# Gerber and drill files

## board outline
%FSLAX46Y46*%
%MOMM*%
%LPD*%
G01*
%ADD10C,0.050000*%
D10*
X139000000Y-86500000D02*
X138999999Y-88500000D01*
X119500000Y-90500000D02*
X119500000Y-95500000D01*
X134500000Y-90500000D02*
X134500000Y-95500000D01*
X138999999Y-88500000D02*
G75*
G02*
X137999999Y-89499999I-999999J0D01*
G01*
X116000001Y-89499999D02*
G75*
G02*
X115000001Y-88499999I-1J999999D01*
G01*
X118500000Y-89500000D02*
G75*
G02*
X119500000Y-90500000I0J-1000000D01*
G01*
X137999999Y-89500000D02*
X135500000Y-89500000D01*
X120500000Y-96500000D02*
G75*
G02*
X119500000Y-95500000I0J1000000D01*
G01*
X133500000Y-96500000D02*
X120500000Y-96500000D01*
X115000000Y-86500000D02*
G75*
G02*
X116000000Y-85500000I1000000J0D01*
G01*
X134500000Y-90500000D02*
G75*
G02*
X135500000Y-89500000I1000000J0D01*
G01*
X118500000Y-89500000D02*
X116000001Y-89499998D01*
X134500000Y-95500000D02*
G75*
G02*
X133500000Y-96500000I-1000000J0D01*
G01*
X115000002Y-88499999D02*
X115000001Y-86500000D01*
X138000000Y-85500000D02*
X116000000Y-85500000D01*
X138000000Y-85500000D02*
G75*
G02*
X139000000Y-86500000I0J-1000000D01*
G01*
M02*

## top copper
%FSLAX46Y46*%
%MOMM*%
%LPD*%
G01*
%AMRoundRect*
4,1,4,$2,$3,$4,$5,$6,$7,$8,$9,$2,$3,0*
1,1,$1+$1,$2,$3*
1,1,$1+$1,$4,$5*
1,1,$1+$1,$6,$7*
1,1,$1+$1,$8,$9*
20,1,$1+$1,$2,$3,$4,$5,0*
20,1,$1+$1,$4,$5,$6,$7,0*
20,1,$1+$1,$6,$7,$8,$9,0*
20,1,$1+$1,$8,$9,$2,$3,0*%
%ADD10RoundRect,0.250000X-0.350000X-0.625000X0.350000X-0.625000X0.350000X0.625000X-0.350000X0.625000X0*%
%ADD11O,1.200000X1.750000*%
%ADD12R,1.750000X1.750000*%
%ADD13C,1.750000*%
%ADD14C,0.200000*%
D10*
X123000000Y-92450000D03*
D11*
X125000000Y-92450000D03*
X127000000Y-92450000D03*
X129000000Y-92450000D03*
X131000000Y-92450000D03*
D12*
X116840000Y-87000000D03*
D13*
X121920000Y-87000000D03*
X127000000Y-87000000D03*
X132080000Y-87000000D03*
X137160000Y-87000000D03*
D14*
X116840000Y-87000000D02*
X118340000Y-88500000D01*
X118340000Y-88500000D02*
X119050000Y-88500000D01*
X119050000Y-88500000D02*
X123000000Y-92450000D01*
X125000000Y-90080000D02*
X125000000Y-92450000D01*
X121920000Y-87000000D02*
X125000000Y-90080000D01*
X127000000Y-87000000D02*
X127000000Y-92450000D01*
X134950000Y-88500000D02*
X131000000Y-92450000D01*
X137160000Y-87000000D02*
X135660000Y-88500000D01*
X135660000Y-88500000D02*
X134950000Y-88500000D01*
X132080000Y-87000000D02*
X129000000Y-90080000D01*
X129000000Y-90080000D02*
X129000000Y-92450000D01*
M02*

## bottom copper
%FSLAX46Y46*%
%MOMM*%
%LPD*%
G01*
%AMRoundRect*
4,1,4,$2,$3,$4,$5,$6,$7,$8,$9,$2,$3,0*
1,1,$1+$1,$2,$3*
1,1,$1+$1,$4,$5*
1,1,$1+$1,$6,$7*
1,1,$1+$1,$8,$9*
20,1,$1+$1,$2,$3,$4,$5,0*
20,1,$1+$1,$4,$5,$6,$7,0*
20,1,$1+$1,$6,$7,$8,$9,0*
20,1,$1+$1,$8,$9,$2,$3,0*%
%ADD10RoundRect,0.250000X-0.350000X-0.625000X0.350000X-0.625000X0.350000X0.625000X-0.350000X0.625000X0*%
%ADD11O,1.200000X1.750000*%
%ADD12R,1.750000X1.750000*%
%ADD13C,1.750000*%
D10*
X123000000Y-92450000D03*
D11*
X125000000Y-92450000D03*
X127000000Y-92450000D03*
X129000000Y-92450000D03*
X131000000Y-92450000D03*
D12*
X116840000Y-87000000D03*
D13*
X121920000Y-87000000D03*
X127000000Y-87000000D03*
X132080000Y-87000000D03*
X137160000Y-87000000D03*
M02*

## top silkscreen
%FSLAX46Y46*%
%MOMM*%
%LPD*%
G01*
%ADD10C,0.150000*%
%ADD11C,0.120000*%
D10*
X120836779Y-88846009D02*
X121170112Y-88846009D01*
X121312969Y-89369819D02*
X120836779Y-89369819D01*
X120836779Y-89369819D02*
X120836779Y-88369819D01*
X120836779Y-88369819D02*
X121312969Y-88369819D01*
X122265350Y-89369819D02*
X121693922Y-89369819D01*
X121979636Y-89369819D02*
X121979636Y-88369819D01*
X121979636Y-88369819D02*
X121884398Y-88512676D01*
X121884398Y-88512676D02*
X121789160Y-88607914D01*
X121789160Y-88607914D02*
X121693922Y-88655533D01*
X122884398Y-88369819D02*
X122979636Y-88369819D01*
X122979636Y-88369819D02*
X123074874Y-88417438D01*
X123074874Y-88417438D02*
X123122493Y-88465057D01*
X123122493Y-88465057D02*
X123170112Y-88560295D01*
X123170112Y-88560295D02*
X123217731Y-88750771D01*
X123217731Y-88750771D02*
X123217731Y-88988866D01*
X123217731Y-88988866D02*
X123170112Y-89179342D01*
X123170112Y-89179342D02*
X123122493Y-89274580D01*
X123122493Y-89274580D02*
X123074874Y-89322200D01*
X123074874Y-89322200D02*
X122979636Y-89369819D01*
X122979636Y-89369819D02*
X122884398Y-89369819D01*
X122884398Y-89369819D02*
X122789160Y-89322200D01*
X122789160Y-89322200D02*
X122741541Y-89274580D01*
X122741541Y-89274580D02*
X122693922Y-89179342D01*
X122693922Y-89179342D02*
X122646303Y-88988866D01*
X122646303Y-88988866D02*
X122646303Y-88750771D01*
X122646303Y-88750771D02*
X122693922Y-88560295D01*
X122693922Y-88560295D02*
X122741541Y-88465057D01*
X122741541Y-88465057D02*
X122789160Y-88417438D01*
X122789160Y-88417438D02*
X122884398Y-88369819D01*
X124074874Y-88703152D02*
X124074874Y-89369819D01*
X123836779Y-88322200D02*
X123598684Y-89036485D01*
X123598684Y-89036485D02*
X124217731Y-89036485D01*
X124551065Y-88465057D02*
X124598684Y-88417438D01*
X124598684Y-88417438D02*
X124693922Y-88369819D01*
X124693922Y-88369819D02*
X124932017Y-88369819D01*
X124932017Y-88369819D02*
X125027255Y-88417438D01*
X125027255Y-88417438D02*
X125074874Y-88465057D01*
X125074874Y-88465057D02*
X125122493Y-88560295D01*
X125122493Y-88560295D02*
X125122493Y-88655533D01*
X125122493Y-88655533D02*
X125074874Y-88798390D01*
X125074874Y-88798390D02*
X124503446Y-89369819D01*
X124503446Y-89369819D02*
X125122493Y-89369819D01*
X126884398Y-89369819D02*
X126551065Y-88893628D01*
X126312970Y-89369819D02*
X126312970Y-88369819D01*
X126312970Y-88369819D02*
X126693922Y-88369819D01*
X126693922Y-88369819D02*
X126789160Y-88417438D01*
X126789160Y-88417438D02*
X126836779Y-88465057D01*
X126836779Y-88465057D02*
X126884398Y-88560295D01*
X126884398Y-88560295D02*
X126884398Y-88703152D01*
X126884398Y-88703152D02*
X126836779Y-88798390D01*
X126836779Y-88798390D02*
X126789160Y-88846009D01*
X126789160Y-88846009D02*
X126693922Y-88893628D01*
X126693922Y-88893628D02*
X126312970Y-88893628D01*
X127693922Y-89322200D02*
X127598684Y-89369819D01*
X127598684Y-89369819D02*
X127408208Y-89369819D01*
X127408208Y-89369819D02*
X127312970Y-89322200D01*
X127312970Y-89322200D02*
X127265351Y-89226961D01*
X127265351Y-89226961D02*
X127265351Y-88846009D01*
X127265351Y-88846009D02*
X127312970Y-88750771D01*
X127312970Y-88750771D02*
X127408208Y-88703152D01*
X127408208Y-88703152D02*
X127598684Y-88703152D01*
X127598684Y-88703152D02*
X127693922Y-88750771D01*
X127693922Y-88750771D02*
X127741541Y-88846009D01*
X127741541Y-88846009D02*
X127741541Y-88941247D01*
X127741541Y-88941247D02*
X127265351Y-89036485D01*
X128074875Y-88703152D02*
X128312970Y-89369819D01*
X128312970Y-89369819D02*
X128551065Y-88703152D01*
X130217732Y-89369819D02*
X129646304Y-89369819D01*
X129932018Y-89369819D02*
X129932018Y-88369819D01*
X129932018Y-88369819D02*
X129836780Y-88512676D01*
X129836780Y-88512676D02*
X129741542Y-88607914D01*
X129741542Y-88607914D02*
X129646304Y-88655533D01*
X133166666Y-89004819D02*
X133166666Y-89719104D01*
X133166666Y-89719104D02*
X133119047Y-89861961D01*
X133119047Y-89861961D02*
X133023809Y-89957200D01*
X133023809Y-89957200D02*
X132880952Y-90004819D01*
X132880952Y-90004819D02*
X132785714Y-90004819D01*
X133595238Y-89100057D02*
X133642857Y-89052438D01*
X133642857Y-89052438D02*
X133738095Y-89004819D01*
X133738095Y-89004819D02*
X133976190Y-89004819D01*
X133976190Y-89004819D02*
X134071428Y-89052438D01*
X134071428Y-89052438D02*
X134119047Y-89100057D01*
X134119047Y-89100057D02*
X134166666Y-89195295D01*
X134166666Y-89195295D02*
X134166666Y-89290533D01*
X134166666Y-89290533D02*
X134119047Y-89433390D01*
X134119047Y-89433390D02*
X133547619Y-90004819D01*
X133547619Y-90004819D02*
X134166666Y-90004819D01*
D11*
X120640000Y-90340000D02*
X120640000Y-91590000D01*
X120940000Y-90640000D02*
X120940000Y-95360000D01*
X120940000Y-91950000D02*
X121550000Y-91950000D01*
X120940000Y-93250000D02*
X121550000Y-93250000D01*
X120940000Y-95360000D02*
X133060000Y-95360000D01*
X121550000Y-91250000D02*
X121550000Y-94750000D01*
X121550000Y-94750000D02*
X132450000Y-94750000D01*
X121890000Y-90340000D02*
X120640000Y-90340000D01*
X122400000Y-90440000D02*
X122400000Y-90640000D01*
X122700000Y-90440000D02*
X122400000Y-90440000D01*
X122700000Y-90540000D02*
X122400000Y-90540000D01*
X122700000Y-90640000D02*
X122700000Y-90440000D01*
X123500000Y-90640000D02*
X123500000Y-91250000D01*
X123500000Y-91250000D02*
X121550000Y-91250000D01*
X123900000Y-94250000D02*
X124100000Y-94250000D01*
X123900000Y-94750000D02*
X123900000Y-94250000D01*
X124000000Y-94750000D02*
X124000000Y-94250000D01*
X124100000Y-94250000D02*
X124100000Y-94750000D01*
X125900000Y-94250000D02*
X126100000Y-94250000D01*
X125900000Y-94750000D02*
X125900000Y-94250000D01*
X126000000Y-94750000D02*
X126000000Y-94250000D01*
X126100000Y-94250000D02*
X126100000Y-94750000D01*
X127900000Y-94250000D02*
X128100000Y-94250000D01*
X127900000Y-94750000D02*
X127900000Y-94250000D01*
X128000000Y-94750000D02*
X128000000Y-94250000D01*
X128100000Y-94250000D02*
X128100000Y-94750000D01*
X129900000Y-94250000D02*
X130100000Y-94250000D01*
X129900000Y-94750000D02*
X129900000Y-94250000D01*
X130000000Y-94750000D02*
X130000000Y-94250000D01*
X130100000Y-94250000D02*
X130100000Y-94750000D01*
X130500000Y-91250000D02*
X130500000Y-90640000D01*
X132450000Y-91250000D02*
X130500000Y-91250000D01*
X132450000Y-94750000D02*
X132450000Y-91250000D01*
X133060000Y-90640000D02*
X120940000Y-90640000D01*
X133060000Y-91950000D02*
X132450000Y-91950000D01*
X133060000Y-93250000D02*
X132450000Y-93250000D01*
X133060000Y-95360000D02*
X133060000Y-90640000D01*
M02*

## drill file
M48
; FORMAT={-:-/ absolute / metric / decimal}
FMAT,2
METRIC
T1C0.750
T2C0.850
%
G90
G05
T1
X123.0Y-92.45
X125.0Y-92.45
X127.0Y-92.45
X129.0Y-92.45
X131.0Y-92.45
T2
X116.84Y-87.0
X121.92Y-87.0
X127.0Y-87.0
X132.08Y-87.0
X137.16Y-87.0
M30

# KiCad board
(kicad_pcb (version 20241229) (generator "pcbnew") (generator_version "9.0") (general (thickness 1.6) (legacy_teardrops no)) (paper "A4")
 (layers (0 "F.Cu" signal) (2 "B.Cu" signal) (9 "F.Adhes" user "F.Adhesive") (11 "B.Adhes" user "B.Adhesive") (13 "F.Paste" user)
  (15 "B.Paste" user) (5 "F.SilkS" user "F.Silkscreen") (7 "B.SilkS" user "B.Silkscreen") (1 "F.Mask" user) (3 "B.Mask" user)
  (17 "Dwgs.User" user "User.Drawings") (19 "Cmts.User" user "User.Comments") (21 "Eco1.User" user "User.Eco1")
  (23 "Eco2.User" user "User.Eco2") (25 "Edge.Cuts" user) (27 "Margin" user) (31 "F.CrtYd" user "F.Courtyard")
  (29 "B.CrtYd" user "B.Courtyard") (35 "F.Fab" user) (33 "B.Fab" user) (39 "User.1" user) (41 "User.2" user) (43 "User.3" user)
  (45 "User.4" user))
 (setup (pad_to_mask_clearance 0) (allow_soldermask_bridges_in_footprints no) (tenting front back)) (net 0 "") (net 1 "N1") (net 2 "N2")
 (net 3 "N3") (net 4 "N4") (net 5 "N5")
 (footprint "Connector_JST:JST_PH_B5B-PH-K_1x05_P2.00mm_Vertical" (layer "F.Cu") (at 123 92.45)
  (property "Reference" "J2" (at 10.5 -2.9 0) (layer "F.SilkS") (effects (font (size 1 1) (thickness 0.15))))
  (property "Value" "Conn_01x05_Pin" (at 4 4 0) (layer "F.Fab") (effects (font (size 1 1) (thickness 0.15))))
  (fp_line (start -2.36 -2.11) (end -2.36 -0.86) (stroke (width 0.12) (type solid)) (layer "F.SilkS"))
  (fp_line (start -2.06 -1.81) (end -2.06 2.91) (stroke (width 0.12) (type solid)) (layer "F.SilkS"))
  (fp_line (start -2.06 -0.5) (end -1.45 -0.5) (stroke (width 0.12) (type solid)) (layer "F.SilkS"))
  (fp_line (start -2.06 0.8) (end -1.45 0.8) (stroke (width 0.12) (type solid)) (layer "F.SilkS"))
  (fp_line (start -2.06 2.91) (end 10.06 2.91) (stroke (width 0.12) (type solid)) (layer "F.SilkS"))
  (fp_line (start -1.45 -1.2) (end -1.45 2.3) (stroke (width 0.12) (type solid)) (layer "F.SilkS"))
  (fp_line (start -1.45 2.3) (end 9.45 2.3) (stroke (width 0.12) (type solid)) (layer "F.SilkS"))
  (fp_line (start -1.11 -2.11) (end -2.36 -2.11) (stroke (width 0.12) (type solid)) (layer "F.SilkS"))
  (fp_line (start -0.6 -2.01) (end -0.6 -1.81) (stroke (width 0.12) (type solid)) (layer "F.SilkS"))
  (fp_line (start -0.3 -2.01) (end -0.6 -2.01) (stroke (width 0.12) (type solid)) (layer "F.SilkS"))
  (fp_line (start -0.3 -1.91) (end -0.6 -1.91) (stroke (width 0.12) (type solid)) (layer "F.SilkS"))
  (fp_line (start -0.3 -1.81) (end -0.3 -2.01) (stroke (width 0.12) (type solid)) (layer "F.SilkS"))
  (fp_line (start 0.5 -1.81) (end 0.5 -1.2) (stroke (width 0.12) (type solid)) (layer "F.SilkS"))
  (fp_line (start 0.5 -1.2) (end -1.45 -1.2) (stroke (width 0.12) (type solid)) (layer "F.SilkS"))
  (fp_line (start 0.9 1.8) (end 1.1 1.8) (stroke (width 0.12) (type solid)) (layer "F.SilkS"))
  (fp_line (start 0.9 2.3) (end 0.9 1.8) (stroke (width 0.12) (type solid)) (layer "F.SilkS"))
  (fp_line (start 1 2.3) (end 1 1.8) (stroke (width 0.12) (type solid)) (layer "F.SilkS"))
  (fp_line (start 1.1 1.8) (end 1.1 2.3) (stroke (width 0.12) (type solid)) (layer "F.SilkS"))
  (fp_line (start 2.9 1.8) (end 3.1 1.8) (stroke (width 0.12) (type solid)) (layer "F.SilkS"))
  (fp_line (start 2.9 2.3) (end 2.9 1.8) (stroke (width 0.12) (type solid)) (layer "F.SilkS"))
  (fp_line (start 3 2.3) (end 3 1.8) (stroke (width 0.12) (type solid)) (layer "F.SilkS"))
  (fp_line (start 3.1 1.8) (end 3.1 2.3) (stroke (width 0.12) (type solid)) (layer "F.SilkS"))
  (fp_line (start 4.9 1.8) (end 5.1 1.8) (stroke (width 0.12) (type solid)) (layer "F.SilkS"))
  (fp_line (start 4.9 2.3) (end 4.9 1.8) (stroke (width 0.12) (type solid)) (layer "F.SilkS"))
  (fp_line (start 5 2.3) (end 5 1.8) (stroke (width 0.12) (type solid)) (layer "F.SilkS"))
  (fp_line (start 5.1 1.8) (end 5.1 2.3) (stroke (width 0.12) (type solid)) (layer "F.SilkS"))
  (fp_line (start 6.9 1.8) (end 7.1 1.8) (stroke (width 0.12) (type solid)) (layer "F.SilkS"))
  (fp_line (start 6.9 2.3) (end 6.9 1.8) (stroke (width 0.12) (type solid)) (layer "F.SilkS"))
  (fp_line (start 7 2.3) (end 7 1.8) (stroke (width 0.12) (type solid)) (layer "F.SilkS"))
  (fp_line (start 7.1 1.8) (end 7.1 2.3) (stroke (width 0.12) (type solid)) (layer "F.SilkS"))
  (fp_line (start 7.5 -1.2) (end 7.5 -1.81) (stroke (width 0.12) (type solid)) (layer "F.SilkS"))
  (fp_line (start 9.45 -1.2) (end 7.5 -1.2) (stroke (width 0.12) (type solid)) (layer "F.SilkS"))
  (fp_line (start 9.45 2.3) (end 9.45 -1.2) (stroke (width 0.12) (type solid)) (layer "F.SilkS"))
  (fp_line (start 10.06 -1.81) (end -2.06 -1.81) (stroke (width 0.12) (type solid)) (layer "F.SilkS"))
  (fp_line (start 10.06 -0.5) (end 9.45 -0.5) (stroke (width 0.12) (type solid)) (layer "F.SilkS"))
  (fp_line (start 10.06 0.8) (end 9.45 0.8) (stroke (width 0.12) (type solid)) (layer "F.SilkS"))
  (fp_line (start 10.06 2.91) (end 10.06 -1.81) (stroke (width 0.12) (type solid)) (layer "F.SilkS"))
  (pad "1" thru_hole roundrect (at 0 0) (size 1.2 1.75) (drill 0.75) (layers "*.Cu" "*.Mask") (remove_unused_layers no)
   (roundrect_rratio 0.208333) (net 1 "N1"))
  (pad "2" thru_hole oval (at 2 0) (size 1.2 1.75) (drill 0.75) (layers "*.Cu" "*.Mask") (remove_unused_layers no) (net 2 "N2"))
  (pad "3" thru_hole oval (at 4 0) (size 1.2 1.75) (drill 0.75) (layers "*.Cu" "*.Mask") (remove_unused_layers no) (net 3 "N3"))
  (pad "4" thru_hole oval (at 6 0) (size 1.2 1.75) (drill 0.75) (layers "*.Cu" "*.Mask") (remove_unused_layers no) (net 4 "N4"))
  (pad "5" thru_hole oval (at 8 0) (size 1.2 1.75) (drill 0.75) (layers "*.Cu" "*.Mask") (remove_unused_layers no) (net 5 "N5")))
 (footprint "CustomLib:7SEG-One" (layer "B.Cu") (at 116.84 87)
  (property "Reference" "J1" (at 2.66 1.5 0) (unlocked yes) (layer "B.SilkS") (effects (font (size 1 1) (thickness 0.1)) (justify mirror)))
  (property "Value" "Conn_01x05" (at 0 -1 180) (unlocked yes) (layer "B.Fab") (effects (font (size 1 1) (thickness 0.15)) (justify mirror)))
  (pad "1" thru_hole rect (at 0 0) (size 1.75 1.75) (drill 0.85) (layers "*.Cu" "*.Mask") (remove_unused_layers no) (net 1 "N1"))
  (pad "2" thru_hole circle (at 5.08 0) (size 1.75 1.75) (drill 0.85) (layers "*.Cu" "*.Mask") (remove_unused_layers no) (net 2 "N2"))
  (pad "3" thru_hole circle (at 10.16 0) (size 1.75 1.75) (drill 0.85) (layers "*.Cu" "*.Mask") (remove_unused_layers no) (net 3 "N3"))
  (pad "4" thru_hole circle (at 15.24 0) (size 1.75 1.75) (drill 0.85) (layers "*.Cu" "*.Mask") (remove_unused_layers no) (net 4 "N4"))
  (pad "5" thru_hole circle (at 20.32 0) (size 1.75 1.75) (drill 0.85) (layers "*.Cu" "*.Mask") (remove_unused_layers no) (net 5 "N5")))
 (gr_line (start 139 86.5) (end 138.999999 88.5) (stroke (width 0.05) (type default)) (layer "Edge.Cuts"))
 (gr_line (start 119.5 90.5) (end 119.5 95.5) (stroke (width 0.05) (type default)) (layer "Edge.Cuts"))
 (gr_line (start 134.5 90.5) (end 134.5 95.5) (stroke (width 0.05) (type default)) (layer "Edge.Cuts"))
 (gr_arc (start 138.999999 88.5) (mid 138.707106 89.207107) (end 137.999999 89.5) (stroke (width 0.05) (type default)) (layer "Edge.Cuts"))
 (gr_arc (start 116.000001 89.499999) (mid 115.292894 89.207106) (end 115.000001 88.499999) (stroke (width 0.05) (type default))
  (layer "Edge.Cuts"))
 (gr_arc (start 118.5 89.5) (mid 119.207107 89.792893) (end 119.5 90.5) (stroke (width 0.05) (type default)) (layer "Edge.Cuts"))
 (gr_line (start 137.999999 89.5) (end 135.5 89.5) (stroke (width 0.05) (type default)) (layer "Edge.Cuts"))
 (gr_arc (start 120.5 96.5) (mid 119.792893 96.207107) (end 119.5 95.5) (stroke (width 0.05) (type default)) (layer "Edge.Cuts"))
 (gr_line (start 133.5 96.5) (end 120.5 96.5) (stroke (width 0.05) (type default)) (layer "Edge.Cuts"))
 (gr_arc (start 115 86.5) (mid 115.292893 85.792893) (end 116 85.5) (stroke (width 0.05) (type default)) (layer "Edge.Cuts"))
 (gr_arc (start 134.5 90.5) (mid 134.792893 89.792893) (end 135.5 89.5) (stroke (width 0.05) (type default)) (layer "Edge.Cuts"))
 (gr_line (start 118.5 89.5) (end 116.000001 89.499998) (stroke (width 0.05) (type default)) (layer "Edge.Cuts"))
 (gr_arc (start 134.5 95.5) (mid 134.207107 96.207107) (end 133.5 96.5) (stroke (width 0.05) (type default)) (layer "Edge.Cuts"))
 (gr_line (start 115.000002 88.499999) (end 115.000001 86.5) (stroke (width 0.05) (type default)) (layer "Edge.Cuts"))
 (gr_line (start 138 85.5) (end 116 85.5) (stroke (width 0.05) (type default)) (layer "Edge.Cuts"))
 (gr_arc (start 138 85.5) (mid 138.707107 85.792893) (end 139 86.5) (stroke (width 0.05) (type default)) (layer "Edge.Cuts"))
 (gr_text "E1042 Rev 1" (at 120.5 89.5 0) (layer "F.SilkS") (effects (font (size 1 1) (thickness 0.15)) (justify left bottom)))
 (segment (start 116.84 87) (end 118.34 88.5) (width 0.2) (layer "F.Cu") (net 1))
 (segment (start 118.34 88.5) (end 119.05 88.5) (width 0.2) (layer "F.Cu") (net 1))
 (segment (start 119.05 88.5) (end 123 92.45) (width 0.2) (layer "F.Cu") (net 1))
 (segment (start 125 90.08) (end 125 92.45) (width 0.2) (layer "F.Cu") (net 2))
 (segment (start 121.92 87) (end 125 90.08) (width 0.2) (layer "F.Cu") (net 2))
 (segment (start 127 87) (end 127 92.45) (width 0.2) (layer "F.Cu") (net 3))
 (segment (start 134.95 88.5) (end 131 92.45) (width 0.2) (layer "F.Cu") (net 5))
 (segment (start 137.16 87) (end 135.66 88.5) (width 0.2) (layer "F.Cu") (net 5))
 (segment (start 135.66 88.5) (end 134.95 88.5) (width 0.2) (layer "F.Cu") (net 5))
 (segment (start 132.08 87) (end 129 90.08) (width 0.2) (layer "F.Cu") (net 4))
 (segment (start 129 90.08) (end 129 92.45) (width 0.2) (layer "F.Cu") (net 4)))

